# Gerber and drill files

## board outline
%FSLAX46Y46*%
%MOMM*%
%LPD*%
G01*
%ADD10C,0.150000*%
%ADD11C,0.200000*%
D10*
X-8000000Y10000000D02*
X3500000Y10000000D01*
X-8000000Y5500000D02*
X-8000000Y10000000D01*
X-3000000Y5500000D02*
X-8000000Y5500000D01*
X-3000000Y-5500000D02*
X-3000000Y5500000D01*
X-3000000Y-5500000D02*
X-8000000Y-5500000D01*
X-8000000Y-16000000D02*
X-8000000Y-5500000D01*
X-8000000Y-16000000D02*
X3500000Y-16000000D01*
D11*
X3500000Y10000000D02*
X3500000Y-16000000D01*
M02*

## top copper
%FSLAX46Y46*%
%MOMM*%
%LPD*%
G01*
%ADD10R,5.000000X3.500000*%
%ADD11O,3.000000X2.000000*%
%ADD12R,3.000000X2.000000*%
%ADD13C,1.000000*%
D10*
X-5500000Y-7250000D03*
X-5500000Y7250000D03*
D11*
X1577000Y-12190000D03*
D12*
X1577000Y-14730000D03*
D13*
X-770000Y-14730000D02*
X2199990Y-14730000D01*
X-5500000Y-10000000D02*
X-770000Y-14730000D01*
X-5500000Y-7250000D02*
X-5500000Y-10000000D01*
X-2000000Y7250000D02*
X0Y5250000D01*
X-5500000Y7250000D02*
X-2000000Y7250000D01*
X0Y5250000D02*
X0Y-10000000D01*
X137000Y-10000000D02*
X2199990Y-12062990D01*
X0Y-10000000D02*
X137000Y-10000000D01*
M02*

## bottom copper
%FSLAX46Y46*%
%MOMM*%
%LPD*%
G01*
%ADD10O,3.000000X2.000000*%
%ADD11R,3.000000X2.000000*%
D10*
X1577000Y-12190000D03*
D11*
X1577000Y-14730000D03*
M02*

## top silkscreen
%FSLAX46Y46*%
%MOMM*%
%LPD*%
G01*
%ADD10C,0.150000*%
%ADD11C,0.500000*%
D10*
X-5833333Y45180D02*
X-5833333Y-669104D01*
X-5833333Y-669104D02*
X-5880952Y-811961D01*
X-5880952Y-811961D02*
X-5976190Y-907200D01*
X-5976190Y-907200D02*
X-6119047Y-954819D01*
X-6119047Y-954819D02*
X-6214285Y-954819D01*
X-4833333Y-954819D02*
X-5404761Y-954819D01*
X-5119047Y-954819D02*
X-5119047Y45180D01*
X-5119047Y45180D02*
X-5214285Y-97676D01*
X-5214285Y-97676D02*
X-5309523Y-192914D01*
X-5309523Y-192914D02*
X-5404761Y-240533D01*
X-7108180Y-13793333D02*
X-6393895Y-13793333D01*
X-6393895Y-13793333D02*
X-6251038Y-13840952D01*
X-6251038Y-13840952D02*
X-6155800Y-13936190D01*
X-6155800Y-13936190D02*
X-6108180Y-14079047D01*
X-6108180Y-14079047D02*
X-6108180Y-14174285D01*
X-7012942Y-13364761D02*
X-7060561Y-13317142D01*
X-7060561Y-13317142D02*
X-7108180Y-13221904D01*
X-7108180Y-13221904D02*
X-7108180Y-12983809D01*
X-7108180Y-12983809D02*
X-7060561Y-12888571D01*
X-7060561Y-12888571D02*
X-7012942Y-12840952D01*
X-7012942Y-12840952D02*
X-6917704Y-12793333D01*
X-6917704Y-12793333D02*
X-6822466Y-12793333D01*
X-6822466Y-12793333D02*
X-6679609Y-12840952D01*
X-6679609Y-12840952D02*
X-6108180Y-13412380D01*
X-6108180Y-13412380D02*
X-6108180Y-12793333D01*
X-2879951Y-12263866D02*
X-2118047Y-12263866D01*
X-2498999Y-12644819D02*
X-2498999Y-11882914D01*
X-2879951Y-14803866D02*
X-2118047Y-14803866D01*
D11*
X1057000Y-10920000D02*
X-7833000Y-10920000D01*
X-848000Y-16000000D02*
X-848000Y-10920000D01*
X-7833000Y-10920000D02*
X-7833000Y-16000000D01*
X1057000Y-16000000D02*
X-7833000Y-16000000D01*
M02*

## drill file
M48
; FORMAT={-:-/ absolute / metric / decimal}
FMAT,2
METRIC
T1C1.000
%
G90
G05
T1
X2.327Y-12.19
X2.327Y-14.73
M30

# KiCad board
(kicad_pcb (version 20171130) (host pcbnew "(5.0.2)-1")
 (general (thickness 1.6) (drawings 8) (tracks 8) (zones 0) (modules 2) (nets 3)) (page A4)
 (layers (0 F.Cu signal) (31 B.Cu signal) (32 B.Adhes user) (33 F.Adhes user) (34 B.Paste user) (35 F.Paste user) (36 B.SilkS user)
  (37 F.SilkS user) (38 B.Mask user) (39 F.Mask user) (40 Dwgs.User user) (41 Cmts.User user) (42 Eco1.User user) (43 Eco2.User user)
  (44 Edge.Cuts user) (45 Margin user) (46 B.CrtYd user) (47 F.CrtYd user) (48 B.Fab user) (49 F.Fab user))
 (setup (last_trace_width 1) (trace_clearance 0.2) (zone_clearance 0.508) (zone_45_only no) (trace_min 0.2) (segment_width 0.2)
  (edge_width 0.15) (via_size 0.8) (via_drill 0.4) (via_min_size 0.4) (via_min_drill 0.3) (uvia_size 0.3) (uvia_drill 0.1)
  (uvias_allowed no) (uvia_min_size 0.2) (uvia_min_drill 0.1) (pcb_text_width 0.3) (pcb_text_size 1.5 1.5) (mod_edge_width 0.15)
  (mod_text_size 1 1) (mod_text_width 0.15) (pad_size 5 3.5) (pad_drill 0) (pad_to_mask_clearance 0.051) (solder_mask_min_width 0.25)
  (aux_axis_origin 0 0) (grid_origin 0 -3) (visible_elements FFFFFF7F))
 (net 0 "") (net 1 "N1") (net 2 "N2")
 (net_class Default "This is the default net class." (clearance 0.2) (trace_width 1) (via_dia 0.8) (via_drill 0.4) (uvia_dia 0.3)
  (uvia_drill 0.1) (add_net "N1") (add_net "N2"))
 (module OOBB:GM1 (layer F.Cu) (at -5.5 0)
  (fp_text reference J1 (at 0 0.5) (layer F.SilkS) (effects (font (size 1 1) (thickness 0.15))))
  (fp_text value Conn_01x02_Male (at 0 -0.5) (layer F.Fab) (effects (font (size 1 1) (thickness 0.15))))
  (pad 1 smd rect (at 0 7.25) (size 5 3.5) (layers F.Cu F.Paste F.Mask) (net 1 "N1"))
  (pad 2 smd rect (at 0 -7.25) (size 5 3.5) (layers F.Cu F.Paste F.Mask) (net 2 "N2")))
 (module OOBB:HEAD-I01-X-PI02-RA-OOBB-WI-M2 (layer F.Cu) (at 2.327 14.73 180)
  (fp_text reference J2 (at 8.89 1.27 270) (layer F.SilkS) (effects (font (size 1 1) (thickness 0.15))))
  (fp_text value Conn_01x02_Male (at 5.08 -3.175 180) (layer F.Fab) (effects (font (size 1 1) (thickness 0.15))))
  (fp_line (start 1.27 3.81) (end 10.16 3.81) (layer F.SilkS) (width 0.5))
  (fp_line (start 3.175 -1.27) (end 3.175 3.81) (layer F.SilkS) (width 0.5))
  (fp_line (start 10.16 3.81) (end 10.16 -1.27) (layer F.SilkS) (width 0.5))
  (fp_line (start 1.27 -1.27) (end 10.16 -1.27) (layer F.SilkS) (width 0.5))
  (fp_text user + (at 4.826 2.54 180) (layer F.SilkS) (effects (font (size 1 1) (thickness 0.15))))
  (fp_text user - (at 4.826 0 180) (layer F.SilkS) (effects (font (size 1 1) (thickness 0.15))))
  (pad 2 thru_hole oval (at 0 2.54 180) (size 3 2) (drill 1 (offset 0.75 0)) (layers *.Cu *.Mask) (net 2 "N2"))
  (pad 1 thru_hole rect (at 0 0 180) (size 3 2) (drill 1 (offset 0.75 0)) (layers *.Cu *.Mask) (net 1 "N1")))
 (gr_line (start -8 -10) (end 3.5 -10) (layer Edge.Cuts) (width 0.15))
 (gr_line (start -8 -5.5) (end -8 -10) (layer Edge.Cuts) (width 0.15))
 (gr_line (start -3 -5.5) (end -8 -5.5) (layer Edge.Cuts) (width 0.15))
 (gr_line (start -3 5.5) (end -3 -5.5) (layer Edge.Cuts) (width 0.15))
 (gr_line (start -3 5.5) (end -8 5.5) (layer Edge.Cuts) (width 0.15))
 (gr_line (start -8 16) (end -8 5.5) (layer Edge.Cuts) (width 0.15))
 (gr_line (start -8 16) (end 3.5 16) (layer Edge.Cuts) (width 0.15))
 (gr_line (start 3.5 -10) (end 3.5 16) (layer Edge.Cuts) (width 0.2))
 (segment (start -0.77 14.73) (end 2.19999 14.73) (width 1) (layer F.Cu) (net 1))
 (segment (start -5.5 10) (end -0.77 14.73) (width 1) (layer F.Cu) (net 1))
 (segment (start -5.5 7.25) (end -5.5 10) (width 1) (layer F.Cu) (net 1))
 (segment (start -2 -7.25) (end 0 -5.25) (width 1) (layer F.Cu) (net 2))
 (segment (start -5.5 -7.25) (end -2 -7.25) (width 1) (layer F.Cu) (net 2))
 (segment (start 0 -5.25) (end 0 10) (width 1) (layer F.Cu) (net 2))
 (segment (start 0.137 10) (end 2.19999 12.06299) (width 1) (layer F.Cu) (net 2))
 (segment (start 0 10) (end 0.137 10) (width 1) (layer F.Cu) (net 2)))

